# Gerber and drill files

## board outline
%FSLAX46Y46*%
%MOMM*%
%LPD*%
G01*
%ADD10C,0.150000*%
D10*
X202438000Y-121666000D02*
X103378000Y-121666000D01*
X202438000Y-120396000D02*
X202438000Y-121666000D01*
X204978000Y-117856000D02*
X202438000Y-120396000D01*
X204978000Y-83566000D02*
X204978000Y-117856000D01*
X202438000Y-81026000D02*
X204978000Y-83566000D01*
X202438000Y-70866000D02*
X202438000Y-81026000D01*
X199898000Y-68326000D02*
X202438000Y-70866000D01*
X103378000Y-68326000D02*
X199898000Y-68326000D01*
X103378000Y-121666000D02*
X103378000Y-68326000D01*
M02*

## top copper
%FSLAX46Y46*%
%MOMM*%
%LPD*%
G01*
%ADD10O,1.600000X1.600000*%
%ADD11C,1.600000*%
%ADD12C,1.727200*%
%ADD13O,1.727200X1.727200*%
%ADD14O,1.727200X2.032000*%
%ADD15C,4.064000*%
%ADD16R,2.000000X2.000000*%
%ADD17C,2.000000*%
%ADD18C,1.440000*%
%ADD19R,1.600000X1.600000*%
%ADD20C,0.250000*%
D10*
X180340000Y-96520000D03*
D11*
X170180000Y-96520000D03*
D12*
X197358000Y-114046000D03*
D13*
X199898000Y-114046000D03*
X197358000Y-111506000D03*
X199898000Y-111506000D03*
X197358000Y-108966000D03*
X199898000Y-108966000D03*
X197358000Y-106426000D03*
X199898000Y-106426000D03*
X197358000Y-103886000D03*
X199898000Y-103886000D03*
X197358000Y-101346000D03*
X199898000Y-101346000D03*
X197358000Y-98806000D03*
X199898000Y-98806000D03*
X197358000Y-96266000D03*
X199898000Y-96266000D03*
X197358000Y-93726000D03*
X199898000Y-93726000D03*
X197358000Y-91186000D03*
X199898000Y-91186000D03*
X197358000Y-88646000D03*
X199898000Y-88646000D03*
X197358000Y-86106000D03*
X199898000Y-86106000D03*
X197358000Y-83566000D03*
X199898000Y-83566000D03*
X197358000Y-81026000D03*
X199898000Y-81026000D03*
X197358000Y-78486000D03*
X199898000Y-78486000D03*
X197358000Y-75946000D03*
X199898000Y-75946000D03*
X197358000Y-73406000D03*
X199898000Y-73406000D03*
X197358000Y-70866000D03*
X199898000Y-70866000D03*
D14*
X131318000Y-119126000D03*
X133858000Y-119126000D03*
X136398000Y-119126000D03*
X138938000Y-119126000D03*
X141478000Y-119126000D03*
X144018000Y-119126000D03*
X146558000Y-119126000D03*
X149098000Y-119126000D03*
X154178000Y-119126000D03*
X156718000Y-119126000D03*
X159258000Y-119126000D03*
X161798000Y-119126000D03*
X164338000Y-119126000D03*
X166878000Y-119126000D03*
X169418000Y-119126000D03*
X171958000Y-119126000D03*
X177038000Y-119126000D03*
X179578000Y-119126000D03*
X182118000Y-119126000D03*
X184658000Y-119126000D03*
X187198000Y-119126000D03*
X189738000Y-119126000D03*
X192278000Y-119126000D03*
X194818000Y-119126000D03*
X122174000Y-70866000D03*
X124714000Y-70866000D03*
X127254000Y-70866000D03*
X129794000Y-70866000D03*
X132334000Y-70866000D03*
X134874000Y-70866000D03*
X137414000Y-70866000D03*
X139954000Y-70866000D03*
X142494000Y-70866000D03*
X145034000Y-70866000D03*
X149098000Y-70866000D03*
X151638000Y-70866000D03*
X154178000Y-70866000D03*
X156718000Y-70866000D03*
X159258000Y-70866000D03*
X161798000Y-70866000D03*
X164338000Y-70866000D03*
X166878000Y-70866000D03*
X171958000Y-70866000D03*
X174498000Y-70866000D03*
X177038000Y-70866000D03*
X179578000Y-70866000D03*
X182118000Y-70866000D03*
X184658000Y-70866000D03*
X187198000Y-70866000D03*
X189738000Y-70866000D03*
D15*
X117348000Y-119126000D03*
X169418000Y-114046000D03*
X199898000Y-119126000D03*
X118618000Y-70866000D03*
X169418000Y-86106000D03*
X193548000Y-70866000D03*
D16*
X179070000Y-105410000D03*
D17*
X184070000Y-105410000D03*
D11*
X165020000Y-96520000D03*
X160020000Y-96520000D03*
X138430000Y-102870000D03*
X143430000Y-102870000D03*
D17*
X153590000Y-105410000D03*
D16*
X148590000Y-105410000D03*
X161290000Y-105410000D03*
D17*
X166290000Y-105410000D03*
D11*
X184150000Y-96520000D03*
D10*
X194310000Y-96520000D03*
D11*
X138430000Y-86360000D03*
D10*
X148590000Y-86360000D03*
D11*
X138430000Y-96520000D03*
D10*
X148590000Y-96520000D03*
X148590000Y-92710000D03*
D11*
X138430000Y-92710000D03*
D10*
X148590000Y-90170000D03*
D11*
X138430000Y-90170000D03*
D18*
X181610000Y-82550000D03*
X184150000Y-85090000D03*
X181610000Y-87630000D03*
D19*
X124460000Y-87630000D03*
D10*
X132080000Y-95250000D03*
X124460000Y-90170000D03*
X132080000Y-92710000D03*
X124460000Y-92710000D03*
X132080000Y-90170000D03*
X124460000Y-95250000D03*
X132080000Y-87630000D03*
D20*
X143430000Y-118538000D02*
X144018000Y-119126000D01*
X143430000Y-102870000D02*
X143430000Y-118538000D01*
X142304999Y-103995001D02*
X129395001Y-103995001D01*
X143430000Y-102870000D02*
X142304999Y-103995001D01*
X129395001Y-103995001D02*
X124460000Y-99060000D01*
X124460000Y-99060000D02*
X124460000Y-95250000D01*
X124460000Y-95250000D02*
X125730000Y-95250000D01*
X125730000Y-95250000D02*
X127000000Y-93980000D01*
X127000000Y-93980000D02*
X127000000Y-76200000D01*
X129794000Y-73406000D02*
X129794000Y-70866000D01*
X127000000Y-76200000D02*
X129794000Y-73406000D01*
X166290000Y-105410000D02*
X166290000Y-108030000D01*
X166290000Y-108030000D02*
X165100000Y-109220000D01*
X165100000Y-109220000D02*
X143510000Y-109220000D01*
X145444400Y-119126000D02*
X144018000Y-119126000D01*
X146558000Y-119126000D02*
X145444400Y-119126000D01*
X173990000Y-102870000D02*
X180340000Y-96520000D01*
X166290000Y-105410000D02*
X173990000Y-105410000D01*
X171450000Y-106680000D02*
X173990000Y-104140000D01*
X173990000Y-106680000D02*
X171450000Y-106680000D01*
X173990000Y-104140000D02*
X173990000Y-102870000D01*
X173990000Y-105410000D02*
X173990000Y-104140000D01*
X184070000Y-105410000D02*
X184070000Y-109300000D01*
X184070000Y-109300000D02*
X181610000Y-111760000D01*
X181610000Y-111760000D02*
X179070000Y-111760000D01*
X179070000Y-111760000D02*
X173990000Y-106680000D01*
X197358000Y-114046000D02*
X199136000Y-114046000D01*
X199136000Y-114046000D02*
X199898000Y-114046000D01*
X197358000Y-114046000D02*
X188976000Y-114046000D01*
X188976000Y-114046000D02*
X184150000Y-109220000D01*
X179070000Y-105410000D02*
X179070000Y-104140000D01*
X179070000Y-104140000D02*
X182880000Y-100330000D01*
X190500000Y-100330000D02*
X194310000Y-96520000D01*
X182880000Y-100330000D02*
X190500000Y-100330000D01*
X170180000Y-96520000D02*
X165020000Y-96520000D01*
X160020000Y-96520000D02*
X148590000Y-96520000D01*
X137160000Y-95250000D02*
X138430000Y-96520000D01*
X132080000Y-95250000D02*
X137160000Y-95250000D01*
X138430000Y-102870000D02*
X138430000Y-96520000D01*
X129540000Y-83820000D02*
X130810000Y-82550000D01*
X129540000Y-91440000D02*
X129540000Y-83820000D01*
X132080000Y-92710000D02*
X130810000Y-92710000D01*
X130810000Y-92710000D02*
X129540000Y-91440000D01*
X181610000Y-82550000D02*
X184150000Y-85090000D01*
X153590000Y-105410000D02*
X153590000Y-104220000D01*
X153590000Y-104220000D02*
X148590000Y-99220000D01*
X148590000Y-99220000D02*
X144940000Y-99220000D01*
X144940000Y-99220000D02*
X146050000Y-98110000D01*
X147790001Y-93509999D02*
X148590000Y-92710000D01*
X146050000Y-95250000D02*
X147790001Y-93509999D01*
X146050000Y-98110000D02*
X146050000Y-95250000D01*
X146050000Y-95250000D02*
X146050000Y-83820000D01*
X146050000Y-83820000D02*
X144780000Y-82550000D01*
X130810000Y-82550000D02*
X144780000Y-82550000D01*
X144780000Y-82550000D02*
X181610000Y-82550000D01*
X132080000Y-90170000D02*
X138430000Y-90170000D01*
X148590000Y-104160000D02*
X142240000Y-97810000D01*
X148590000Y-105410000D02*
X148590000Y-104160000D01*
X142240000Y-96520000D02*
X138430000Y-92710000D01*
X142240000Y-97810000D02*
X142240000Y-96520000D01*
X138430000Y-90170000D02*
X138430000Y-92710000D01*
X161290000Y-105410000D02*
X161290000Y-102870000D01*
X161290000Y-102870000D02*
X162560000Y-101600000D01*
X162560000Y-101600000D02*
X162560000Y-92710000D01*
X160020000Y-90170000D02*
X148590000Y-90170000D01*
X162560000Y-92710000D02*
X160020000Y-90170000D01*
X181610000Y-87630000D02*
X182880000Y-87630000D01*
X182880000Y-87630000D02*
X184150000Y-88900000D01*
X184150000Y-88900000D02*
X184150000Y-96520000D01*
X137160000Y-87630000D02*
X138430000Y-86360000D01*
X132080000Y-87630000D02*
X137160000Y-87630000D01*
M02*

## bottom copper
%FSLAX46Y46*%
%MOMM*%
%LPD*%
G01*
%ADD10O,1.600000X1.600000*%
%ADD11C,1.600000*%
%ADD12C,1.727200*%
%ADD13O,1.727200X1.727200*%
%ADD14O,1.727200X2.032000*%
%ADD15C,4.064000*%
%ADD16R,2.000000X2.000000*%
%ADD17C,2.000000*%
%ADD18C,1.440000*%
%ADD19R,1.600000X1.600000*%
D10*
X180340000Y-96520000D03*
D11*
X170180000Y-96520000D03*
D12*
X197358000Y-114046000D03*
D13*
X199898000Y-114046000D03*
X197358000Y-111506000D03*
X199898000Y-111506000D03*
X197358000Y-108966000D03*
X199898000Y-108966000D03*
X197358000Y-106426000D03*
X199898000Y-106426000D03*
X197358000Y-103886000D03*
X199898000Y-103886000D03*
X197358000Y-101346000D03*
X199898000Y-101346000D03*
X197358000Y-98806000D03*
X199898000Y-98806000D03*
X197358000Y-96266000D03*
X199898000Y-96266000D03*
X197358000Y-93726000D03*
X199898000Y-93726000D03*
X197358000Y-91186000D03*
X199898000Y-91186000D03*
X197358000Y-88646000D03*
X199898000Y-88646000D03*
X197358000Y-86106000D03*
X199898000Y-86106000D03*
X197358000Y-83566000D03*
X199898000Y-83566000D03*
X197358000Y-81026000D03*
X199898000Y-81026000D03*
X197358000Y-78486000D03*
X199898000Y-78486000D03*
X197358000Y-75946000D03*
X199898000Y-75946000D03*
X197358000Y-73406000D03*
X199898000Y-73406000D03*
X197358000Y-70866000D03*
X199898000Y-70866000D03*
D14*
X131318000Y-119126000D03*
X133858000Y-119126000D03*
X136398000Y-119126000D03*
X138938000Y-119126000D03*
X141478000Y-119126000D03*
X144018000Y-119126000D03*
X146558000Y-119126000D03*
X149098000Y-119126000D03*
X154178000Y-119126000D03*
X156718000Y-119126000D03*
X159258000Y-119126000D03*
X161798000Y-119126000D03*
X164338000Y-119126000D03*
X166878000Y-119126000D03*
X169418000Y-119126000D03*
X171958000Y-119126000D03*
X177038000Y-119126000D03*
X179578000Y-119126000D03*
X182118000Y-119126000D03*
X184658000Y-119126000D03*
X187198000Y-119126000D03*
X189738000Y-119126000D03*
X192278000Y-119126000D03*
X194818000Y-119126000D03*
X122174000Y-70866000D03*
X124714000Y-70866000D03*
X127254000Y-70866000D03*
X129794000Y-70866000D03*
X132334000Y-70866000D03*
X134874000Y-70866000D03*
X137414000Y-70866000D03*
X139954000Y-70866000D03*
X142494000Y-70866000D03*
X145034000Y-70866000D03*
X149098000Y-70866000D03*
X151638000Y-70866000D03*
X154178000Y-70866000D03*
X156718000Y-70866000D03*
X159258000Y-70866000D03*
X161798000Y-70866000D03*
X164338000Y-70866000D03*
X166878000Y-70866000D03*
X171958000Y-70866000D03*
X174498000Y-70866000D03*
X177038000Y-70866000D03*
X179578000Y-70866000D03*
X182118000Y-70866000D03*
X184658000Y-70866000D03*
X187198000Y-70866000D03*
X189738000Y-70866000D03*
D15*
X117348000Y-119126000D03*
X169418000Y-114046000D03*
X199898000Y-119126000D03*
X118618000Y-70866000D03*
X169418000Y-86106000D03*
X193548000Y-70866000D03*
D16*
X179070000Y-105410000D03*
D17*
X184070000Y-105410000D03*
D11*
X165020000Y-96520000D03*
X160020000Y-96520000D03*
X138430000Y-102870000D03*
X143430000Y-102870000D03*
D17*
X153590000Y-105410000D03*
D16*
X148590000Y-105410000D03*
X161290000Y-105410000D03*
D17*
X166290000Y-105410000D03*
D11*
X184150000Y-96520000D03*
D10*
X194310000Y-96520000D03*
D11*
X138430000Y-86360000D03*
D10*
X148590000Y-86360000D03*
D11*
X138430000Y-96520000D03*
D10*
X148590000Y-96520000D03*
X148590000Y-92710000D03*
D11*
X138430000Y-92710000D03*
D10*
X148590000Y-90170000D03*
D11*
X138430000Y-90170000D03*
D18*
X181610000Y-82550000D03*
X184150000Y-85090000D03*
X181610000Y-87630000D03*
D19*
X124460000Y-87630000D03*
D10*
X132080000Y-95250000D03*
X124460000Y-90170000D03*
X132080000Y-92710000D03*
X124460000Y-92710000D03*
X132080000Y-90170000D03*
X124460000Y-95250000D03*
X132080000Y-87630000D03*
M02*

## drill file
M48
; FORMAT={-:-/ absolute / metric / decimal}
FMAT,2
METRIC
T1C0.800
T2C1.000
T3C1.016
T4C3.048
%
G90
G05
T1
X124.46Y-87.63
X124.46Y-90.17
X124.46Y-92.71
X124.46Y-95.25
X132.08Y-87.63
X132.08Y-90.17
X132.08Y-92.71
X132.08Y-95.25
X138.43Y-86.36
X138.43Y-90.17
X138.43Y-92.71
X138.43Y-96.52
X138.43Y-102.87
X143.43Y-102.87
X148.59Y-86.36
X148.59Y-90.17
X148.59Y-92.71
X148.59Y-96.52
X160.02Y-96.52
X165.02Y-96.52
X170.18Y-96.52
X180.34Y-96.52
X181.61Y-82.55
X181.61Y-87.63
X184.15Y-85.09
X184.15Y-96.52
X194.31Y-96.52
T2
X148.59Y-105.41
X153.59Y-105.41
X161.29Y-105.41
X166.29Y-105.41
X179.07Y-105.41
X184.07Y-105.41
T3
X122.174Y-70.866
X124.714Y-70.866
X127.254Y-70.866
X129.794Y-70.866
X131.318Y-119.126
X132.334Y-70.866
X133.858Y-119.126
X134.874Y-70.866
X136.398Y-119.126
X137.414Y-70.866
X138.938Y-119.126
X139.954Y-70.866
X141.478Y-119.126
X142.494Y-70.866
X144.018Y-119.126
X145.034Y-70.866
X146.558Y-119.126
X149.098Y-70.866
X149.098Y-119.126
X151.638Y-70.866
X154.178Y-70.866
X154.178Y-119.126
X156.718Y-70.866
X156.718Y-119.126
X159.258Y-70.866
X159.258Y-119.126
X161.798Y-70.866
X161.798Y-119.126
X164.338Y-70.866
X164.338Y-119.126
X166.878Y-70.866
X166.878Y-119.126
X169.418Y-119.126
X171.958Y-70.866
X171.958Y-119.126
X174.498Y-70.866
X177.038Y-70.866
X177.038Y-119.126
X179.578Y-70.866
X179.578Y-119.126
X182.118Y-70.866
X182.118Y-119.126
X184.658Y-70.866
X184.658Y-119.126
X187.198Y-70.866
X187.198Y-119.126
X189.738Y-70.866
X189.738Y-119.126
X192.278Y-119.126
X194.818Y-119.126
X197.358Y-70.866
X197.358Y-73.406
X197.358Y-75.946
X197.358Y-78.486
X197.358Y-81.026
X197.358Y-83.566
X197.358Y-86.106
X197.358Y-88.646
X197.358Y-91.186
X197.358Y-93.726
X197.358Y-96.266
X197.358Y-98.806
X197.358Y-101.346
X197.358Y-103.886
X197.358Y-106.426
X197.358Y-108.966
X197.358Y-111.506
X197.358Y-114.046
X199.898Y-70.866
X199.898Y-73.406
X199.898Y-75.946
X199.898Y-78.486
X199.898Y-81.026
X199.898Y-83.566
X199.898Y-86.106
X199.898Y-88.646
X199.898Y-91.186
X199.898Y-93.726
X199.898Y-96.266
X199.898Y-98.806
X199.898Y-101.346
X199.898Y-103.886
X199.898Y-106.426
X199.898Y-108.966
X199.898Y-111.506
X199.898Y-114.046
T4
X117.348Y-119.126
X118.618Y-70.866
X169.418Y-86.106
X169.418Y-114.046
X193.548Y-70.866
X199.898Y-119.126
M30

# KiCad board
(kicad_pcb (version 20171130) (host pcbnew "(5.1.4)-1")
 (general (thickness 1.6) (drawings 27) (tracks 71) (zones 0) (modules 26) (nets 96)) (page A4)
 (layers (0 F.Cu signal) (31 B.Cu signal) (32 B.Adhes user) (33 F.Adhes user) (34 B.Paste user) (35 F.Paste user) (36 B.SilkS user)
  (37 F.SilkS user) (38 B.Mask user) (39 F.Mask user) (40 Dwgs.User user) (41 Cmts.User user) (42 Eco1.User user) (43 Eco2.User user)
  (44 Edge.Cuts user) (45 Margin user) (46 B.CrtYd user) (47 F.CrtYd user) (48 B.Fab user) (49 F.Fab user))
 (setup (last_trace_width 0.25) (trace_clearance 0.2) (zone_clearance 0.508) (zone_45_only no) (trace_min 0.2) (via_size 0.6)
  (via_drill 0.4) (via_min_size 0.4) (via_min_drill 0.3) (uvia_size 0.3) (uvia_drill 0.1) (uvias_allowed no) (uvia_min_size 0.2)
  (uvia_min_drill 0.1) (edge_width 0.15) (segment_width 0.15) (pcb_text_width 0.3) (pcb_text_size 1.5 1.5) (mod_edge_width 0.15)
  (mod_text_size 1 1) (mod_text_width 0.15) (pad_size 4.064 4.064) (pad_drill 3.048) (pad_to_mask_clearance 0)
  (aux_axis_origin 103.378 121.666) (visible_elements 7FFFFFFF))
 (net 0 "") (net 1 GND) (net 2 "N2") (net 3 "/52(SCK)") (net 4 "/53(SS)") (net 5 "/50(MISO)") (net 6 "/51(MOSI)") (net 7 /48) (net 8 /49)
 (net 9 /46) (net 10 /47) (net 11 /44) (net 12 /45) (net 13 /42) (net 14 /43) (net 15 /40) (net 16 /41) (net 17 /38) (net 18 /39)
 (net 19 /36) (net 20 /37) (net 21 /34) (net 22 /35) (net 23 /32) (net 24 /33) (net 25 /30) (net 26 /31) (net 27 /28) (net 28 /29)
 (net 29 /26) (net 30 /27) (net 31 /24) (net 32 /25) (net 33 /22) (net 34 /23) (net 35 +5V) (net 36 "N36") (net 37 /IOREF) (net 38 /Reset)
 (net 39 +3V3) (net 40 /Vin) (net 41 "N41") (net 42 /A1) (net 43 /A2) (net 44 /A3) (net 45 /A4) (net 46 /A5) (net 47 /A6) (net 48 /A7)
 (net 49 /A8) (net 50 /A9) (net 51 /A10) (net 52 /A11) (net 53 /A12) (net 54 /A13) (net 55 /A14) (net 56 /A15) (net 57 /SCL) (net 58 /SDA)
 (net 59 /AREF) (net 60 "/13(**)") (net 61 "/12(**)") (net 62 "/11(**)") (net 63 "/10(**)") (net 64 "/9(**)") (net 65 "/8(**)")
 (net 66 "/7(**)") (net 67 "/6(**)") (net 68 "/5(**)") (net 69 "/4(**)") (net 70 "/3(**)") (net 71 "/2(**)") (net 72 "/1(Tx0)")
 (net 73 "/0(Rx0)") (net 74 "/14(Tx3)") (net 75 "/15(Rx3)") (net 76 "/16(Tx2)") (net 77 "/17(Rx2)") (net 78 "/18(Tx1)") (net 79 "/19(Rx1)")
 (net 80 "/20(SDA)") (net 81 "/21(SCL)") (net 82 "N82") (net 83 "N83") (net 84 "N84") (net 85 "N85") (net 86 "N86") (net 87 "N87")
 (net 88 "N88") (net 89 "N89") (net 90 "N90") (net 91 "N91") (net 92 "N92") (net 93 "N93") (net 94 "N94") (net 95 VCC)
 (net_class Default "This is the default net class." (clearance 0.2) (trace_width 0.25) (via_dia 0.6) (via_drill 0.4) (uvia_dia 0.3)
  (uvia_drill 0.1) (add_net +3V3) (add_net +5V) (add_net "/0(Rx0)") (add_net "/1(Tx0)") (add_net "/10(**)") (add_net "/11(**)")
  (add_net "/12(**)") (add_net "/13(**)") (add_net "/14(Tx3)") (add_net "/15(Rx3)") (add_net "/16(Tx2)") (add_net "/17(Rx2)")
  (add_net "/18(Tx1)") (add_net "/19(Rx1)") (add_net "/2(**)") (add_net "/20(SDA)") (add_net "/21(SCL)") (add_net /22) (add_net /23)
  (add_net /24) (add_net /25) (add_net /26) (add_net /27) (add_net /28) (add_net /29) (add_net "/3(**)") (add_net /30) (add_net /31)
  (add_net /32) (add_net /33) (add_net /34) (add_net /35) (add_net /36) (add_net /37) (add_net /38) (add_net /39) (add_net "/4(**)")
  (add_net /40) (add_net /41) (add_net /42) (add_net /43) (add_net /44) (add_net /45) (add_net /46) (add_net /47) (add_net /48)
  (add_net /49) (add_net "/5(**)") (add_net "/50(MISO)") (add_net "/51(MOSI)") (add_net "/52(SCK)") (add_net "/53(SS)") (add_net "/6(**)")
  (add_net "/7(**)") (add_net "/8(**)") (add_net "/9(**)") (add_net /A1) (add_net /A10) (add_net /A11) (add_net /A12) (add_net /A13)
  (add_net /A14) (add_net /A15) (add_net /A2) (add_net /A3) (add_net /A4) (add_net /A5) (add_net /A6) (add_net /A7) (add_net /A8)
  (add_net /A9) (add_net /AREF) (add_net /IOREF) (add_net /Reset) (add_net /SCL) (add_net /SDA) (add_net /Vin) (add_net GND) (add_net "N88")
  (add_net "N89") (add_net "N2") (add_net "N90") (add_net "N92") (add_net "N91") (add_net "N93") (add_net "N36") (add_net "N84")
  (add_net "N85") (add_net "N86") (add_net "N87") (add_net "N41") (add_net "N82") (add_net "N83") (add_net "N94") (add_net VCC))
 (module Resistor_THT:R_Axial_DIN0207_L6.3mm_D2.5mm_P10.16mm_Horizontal (layer F.Cu) (at 170.18 96.52)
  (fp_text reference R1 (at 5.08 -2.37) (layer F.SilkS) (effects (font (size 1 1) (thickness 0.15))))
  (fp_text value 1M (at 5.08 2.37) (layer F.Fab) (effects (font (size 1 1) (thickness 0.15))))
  (pad 2 thru_hole oval (at 10.16 0) (size 1.6 1.6) (drill 0.8) (layers *.Cu *.Mask) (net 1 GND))
  (pad 1 thru_hole circle (at 0 0) (size 1.6 1.6) (drill 0.8) (layers *.Cu *.Mask) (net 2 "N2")))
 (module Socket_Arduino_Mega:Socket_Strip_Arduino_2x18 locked (layer F.Cu) (at 197.358 114.046 90)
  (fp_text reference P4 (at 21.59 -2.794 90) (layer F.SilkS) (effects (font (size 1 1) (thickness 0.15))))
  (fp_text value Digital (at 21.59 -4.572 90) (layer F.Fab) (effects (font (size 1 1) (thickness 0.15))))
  (pad 1 thru_hole circle (at 0 0 90) (size 1.7272 1.7272) (drill 1.016) (layers *.Cu *.Mask F.SilkS) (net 1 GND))
  (pad 2 thru_hole oval (at 0 2.54 90) (size 1.7272 1.7272) (drill 1.016) (layers *.Cu *.Mask F.SilkS) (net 1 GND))
  (pad 3 thru_hole oval (at 2.54 0 90) (size 1.7272 1.7272) (drill 1.016) (layers *.Cu *.Mask F.SilkS) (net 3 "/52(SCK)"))
  (pad 4 thru_hole oval (at 2.54 2.54 90) (size 1.7272 1.7272) (drill 1.016) (layers *.Cu *.Mask F.SilkS) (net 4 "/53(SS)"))
  (pad 5 thru_hole oval (at 5.08 0 90) (size 1.7272 1.7272) (drill 1.016) (layers *.Cu *.Mask F.SilkS) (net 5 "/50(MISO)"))
  (pad 6 thru_hole oval (at 5.08 2.54 90) (size 1.7272 1.7272) (drill 1.016) (layers *.Cu *.Mask F.SilkS) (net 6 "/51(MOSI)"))
  (pad 7 thru_hole oval (at 7.62 0 90) (size 1.7272 1.7272) (drill 1.016) (layers *.Cu *.Mask F.SilkS) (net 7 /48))
  (pad 8 thru_hole oval (at 7.62 2.54 90) (size 1.7272 1.7272) (drill 1.016) (layers *.Cu *.Mask F.SilkS) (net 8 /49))
  (pad 9 thru_hole oval (at 10.16 0 90) (size 1.7272 1.7272) (drill 1.016) (layers *.Cu *.Mask F.SilkS) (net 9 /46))
  (pad 10 thru_hole oval (at 10.16 2.54 90) (size 1.7272 1.7272) (drill 1.016) (layers *.Cu *.Mask F.SilkS) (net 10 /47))
  (pad 11 thru_hole oval (at 12.7 0 90) (size 1.7272 1.7272) (drill 1.016) (layers *.Cu *.Mask F.SilkS) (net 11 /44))
  (pad 12 thru_hole oval (at 12.7 2.54 90) (size 1.7272 1.7272) (drill 1.016) (layers *.Cu *.Mask F.SilkS) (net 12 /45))
  (pad 13 thru_hole oval (at 15.24 0 90) (size 1.7272 1.7272) (drill 1.016) (layers *.Cu *.Mask F.SilkS) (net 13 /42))
  (pad 14 thru_hole oval (at 15.24 2.54 90) (size 1.7272 1.7272) (drill 1.016) (layers *.Cu *.Mask F.SilkS) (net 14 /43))
  (pad 15 thru_hole oval (at 17.78 0 90) (size 1.7272 1.7272) (drill 1.016) (layers *.Cu *.Mask F.SilkS) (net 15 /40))
  (pad 16 thru_hole oval (at 17.78 2.54 90) (size 1.7272 1.7272) (drill 1.016) (layers *.Cu *.Mask F.SilkS) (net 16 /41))
  (pad 17 thru_hole oval (at 20.32 0 90) (size 1.7272 1.7272) (drill 1.016) (layers *.Cu *.Mask F.SilkS) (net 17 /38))
  (pad 18 thru_hole oval (at 20.32 2.54 90) (size 1.7272 1.7272) (drill 1.016) (layers *.Cu *.Mask F.SilkS) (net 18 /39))
  (pad 19 thru_hole oval (at 22.86 0 90) (size 1.7272 1.7272) (drill 1.016) (layers *.Cu *.Mask F.SilkS) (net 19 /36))
  (pad 20 thru_hole oval (at 22.86 2.54 90) (size 1.7272 1.7272) (drill 1.016) (layers *.Cu *.Mask F.SilkS) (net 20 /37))
  (pad 21 thru_hole oval (at 25.4 0 90) (size 1.7272 1.7272) (drill 1.016) (layers *.Cu *.Mask F.SilkS) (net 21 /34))
  (pad 22 thru_hole oval (at 25.4 2.54 90) (size 1.7272 1.7272) (drill 1.016) (layers *.Cu *.Mask F.SilkS) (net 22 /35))
  (pad 23 thru_hole oval (at 27.94 0 90) (size 1.7272 1.7272) (drill 1.016) (layers *.Cu *.Mask F.SilkS) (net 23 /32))
  (pad 24 thru_hole oval (at 27.94 2.54 90) (size 1.7272 1.7272) (drill 1.016) (layers *.Cu *.Mask F.SilkS) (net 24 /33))
  (pad 25 thru_hole oval (at 30.48 0 90) (size 1.7272 1.7272) (drill 1.016) (layers *.Cu *.Mask F.SilkS) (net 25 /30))
  (pad 26 thru_hole oval (at 30.48 2.54 90) (size 1.7272 1.7272) (drill 1.016) (layers *.Cu *.Mask F.SilkS) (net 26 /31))
  (pad 27 thru_hole oval (at 33.02 0 90) (size 1.7272 1.7272) (drill 1.016) (layers *.Cu *.Mask F.SilkS) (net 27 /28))
  (pad 28 thru_hole oval (at 33.02 2.54 90) (size 1.7272 1.7272) (drill 1.016) (layers *.Cu *.Mask F.SilkS) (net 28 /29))
  (pad 29 thru_hole oval (at 35.56 0 90) (size 1.7272 1.7272) (drill 1.016) (layers *.Cu *.Mask F.SilkS) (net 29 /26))
  (pad 30 thru_hole oval (at 35.56 2.54 90) (size 1.7272 1.7272) (drill 1.016) (layers *.Cu *.Mask F.SilkS) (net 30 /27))
  (pad 31 thru_hole oval (at 38.1 0 90) (size 1.7272 1.7272) (drill 1.016) (layers *.Cu *.Mask F.SilkS) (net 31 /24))
  (pad 32 thru_hole oval (at 38.1 2.54 90) (size 1.7272 1.7272) (drill 1.016) (layers *.Cu *.Mask F.SilkS) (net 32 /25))
  (pad 33 thru_hole oval (at 40.64 0 90) (size 1.7272 1.7272) (drill 1.016) (layers *.Cu *.Mask F.SilkS) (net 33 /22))
  (pad 34 thru_hole oval (at 40.64 2.54 90) (size 1.7272 1.7272) (drill 1.016) (layers *.Cu *.Mask F.SilkS) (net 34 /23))
  (pad 35 thru_hole oval (at 43.18 0 90) (size 1.7272 1.7272) (drill 1.016) (layers *.Cu *.Mask F.SilkS) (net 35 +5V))
  (pad 36 thru_hole oval (at 43.18 2.54 90) (size 1.7272 1.7272) (drill 1.016) (layers *.Cu *.Mask F.SilkS) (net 35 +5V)))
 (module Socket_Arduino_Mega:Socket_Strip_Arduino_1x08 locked (layer F.Cu) (at 131.318 119.126)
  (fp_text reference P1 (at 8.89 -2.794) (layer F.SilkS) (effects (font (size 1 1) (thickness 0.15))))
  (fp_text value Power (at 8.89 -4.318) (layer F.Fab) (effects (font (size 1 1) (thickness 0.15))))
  (pad 1 thru_hole oval (at 0 0) (size 1.7272 2.032) (drill 1.016) (layers *.Cu *.Mask F.SilkS) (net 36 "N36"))
  (pad 2 thru_hole oval (at 2.54 0) (size 1.7272 2.032) (drill 1.016) (layers *.Cu *.Mask F.SilkS) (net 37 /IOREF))
  (pad 3 thru_hole oval (at 5.08 0) (size 1.7272 2.032) (drill 1.016) (layers *.Cu *.Mask F.SilkS) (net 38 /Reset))
  (pad 4 thru_hole oval (at 7.62 0) (size 1.7272 2.032) (drill 1.016) (layers *.Cu *.Mask F.SilkS) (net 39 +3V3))
  (pad 5 thru_hole oval (at 10.16 0) (size 1.7272 2.032) (drill 1.016) (layers *.Cu *.Mask F.SilkS) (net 35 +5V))
  (pad 6 thru_hole oval (at 12.7 0) (size 1.7272 2.032) (drill 1.016) (layers *.Cu *.Mask F.SilkS) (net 1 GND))
  (pad 7 thru_hole oval (at 15.24 0) (size 1.7272 2.032) (drill 1.016) (layers *.Cu *.Mask F.SilkS) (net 1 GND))
  (pad 8 thru_hole oval (at 17.78 0) (size 1.7272 2.032) (drill 1.016) (layers *.Cu *.Mask F.SilkS) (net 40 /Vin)))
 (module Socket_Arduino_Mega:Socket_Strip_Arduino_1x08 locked (layer F.Cu) (at 154.178 119.126)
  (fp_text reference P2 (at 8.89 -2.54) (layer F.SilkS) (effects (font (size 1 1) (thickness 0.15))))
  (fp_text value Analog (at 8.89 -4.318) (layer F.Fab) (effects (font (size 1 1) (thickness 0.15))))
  (pad 1 thru_hole oval (at 0 0) (size 1.7272 2.032) (drill 1.016) (layers *.Cu *.Mask F.SilkS) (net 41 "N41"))
  (pad 2 thru_hole oval (at 2.54 0) (size 1.7272 2.032) (drill 1.016) (layers *.Cu *.Mask F.SilkS) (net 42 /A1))
  (pad 3 thru_hole oval (at 5.08 0) (size 1.7272 2.032) (drill 1.016) (layers *.Cu *.Mask F.SilkS) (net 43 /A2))
  (pad 4 thru_hole oval (at 7.62 0) (size 1.7272 2.032) (drill 1.016) (layers *.Cu *.Mask F.SilkS) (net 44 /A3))
  (pad 5 thru_hole oval (at 10.16 0) (size 1.7272 2.032) (drill 1.016) (layers *.Cu *.Mask F.SilkS) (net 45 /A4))
  (pad 6 thru_hole oval (at 12.7 0) (size 1.7272 2.032) (drill 1.016) (layers *.Cu *.Mask F.SilkS) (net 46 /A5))
  (pad 7 thru_hole oval (at 15.24 0) (size 1.7272 2.032) (drill 1.016) (layers *.Cu *.Mask F.SilkS) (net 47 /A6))
  (pad 8 thru_hole oval (at 17.78 0) (size 1.7272 2.032) (drill 1.016) (layers *.Cu *.Mask F.SilkS) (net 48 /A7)))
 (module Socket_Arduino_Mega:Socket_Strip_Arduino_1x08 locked (layer F.Cu) (at 177.038 119.126)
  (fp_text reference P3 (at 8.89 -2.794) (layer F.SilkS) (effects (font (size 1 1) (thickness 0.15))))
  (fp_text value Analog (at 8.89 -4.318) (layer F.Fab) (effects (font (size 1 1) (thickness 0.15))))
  (pad 1 thru_hole oval (at 0 0) (size 1.7272 2.032) (drill 1.016) (layers *.Cu *.Mask F.SilkS) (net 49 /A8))
  (pad 2 thru_hole oval (at 2.54 0) (size 1.7272 2.032) (drill 1.016) (layers *.Cu *.Mask F.SilkS) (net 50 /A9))
  (pad 3 thru_hole oval (at 5.08 0) (size 1.7272 2.032) (drill 1.016) (layers *.Cu *.Mask F.SilkS) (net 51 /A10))
  (pad 4 thru_hole oval (at 7.62 0) (size 1.7272 2.032) (drill 1.016) (layers *.Cu *.Mask F.SilkS) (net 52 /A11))
  (pad 5 thru_hole oval (at 10.16 0) (size 1.7272 2.032) (drill 1.016) (layers *.Cu *.Mask F.SilkS) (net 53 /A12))
  (pad 6 thru_hole oval (at 12.7 0) (size 1.7272 2.032) (drill 1.016) (layers *.Cu *.Mask F.SilkS) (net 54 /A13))
  (pad 7 thru_hole oval (at 15.24 0) (size 1.7272 2.032) (drill 1.016) (layers *.Cu *.Mask F.SilkS) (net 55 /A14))
  (pad 8 thru_hole oval (at 17.78 0) (size 1.7272 2.032) (drill 1.016) (layers *.Cu *.Mask F.SilkS) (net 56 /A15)))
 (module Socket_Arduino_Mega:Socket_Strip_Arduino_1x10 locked (layer F.Cu) (at 122.174 70.866)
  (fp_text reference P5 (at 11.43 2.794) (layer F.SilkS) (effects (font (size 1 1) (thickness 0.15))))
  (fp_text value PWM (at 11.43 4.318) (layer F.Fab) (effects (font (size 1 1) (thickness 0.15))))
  (pad 1 thru_hole oval (at 0 0) (size 1.7272 2.032) (drill 1.016) (layers *.Cu *.Mask F.SilkS) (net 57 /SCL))
  (pad 2 thru_hole oval (at 2.54 0) (size 1.7272 2.032) (drill 1.016) (layers *.Cu *.Mask F.SilkS) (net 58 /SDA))
  (pad 3 thru_hole oval (at 5.08 0) (size 1.7272 2.032) (drill 1.016) (layers *.Cu *.Mask F.SilkS) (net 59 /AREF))
  (pad 4 thru_hole oval (at 7.62 0) (size 1.7272 2.032) (drill 1.016) (layers *.Cu *.Mask F.SilkS) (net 1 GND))
  (pad 5 thru_hole oval (at 10.16 0) (size 1.7272 2.032) (drill 1.016) (layers *.Cu *.Mask F.SilkS) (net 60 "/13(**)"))
  (pad 6 thru_hole oval (at 12.7 0) (size 1.7272 2.032) (drill 1.016) (layers *.Cu *.Mask F.SilkS) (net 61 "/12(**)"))
  (pad 7 thru_hole oval (at 15.24 0) (size 1.7272 2.032) (drill 1.016) (layers *.Cu *.Mask F.SilkS) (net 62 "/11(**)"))
  (pad 8 thru_hole oval (at 17.78 0) (size 1.7272 2.032) (drill 1.016) (layers *.Cu *.Mask F.SilkS) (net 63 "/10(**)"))
  (pad 9 thru_hole oval (at 20.32 0) (size 1.7272 2.032) (drill 1.016) (layers *.Cu *.Mask F.SilkS) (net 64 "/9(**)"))
  (pad 10 thru_hole oval (at 22.86 0) (size 1.7272 2.032) (drill 1.016) (layers *.Cu *.Mask F.SilkS) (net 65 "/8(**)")))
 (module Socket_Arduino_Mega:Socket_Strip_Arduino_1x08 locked (layer F.Cu) (at 149.098 70.866)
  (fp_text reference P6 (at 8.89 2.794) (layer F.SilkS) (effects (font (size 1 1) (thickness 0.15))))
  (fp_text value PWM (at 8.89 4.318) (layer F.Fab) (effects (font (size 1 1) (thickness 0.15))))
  (pad 1 thru_hole oval (at 0 0) (size 1.7272 2.032) (drill 1.016) (layers *.Cu *.Mask F.SilkS) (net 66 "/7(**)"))
  (pad 2 thru_hole oval (at 2.54 0) (size 1.7272 2.032) (drill 1.016) (layers *.Cu *.Mask F.SilkS) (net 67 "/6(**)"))
  (pad 3 thru_hole oval (at 5.08 0) (size 1.7272 2.032) (drill 1.016) (layers *.Cu *.Mask F.SilkS) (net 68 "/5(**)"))
  (pad 4 thru_hole oval (at 7.62 0) (size 1.7272 2.032) (drill 1.016) (layers *.Cu *.Mask F.SilkS) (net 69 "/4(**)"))
  (pad 5 thru_hole oval (at 10.16 0) (size 1.7272 2.032) (drill 1.016) (layers *.Cu *.Mask F.SilkS) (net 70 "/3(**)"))
  (pad 6 thru_hole oval (at 12.7 0) (size 1.7272 2.032) (drill 1.016) (layers *.Cu *.Mask F.SilkS) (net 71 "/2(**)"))
  (pad 7 thru_hole oval (at 15.24 0) (size 1.7272 2.032) (drill 1.016) (layers *.Cu *.Mask F.SilkS) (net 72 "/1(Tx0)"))
  (pad 8 thru_hole oval (at 17.78 0) (size 1.7272 2.032) (drill 1.016) (layers *.Cu *.Mask F.SilkS) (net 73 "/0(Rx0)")))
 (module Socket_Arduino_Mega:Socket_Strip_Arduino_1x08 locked (layer F.Cu) (at 171.958 70.866)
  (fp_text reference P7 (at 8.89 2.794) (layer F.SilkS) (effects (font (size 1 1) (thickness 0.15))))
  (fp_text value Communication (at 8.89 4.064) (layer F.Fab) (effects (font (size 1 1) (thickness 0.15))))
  (pad 1 thru_hole oval (at 0 0) (size 1.7272 2.032) (drill 1.016) (layers *.Cu *.Mask F.SilkS) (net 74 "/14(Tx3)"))
  (pad 2 thru_hole oval (at 2.54 0) (size 1.7272 2.032) (drill 1.016) (layers *.Cu *.Mask F.SilkS) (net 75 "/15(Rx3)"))
  (pad 3 thru_hole oval (at 5.08 0) (size 1.7272 2.032) (drill 1.016) (layers *.Cu *.Mask F.SilkS) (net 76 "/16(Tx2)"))
  (pad 4 thru_hole oval (at 7.62 0) (size 1.7272 2.032) (drill 1.016) (layers *.Cu *.Mask F.SilkS) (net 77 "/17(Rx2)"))
  (pad 5 thru_hole oval (at 10.16 0) (size 1.7272 2.032) (drill 1.016) (layers *.Cu *.Mask F.SilkS) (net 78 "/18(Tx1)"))
  (pad 6 thru_hole oval (at 12.7 0) (size 1.7272 2.032) (drill 1.016) (layers *.Cu *.Mask F.SilkS) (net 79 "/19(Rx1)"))
  (pad 7 thru_hole oval (at 15.24 0) (size 1.7272 2.032) (drill 1.016) (layers *.Cu *.Mask F.SilkS) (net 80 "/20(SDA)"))
  (pad 8 thru_hole oval (at 17.78 0) (size 1.7272 2.032) (drill 1.016) (layers *.Cu *.Mask F.SilkS) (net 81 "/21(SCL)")))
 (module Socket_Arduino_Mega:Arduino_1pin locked (layer F.Cu) (at 117.348 119.126)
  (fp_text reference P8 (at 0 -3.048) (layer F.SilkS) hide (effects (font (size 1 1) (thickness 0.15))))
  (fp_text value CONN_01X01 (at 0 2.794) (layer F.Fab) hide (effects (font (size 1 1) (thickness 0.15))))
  (pad 1 thru_hole circle (at 0 0) (size 4.064 4.064) (drill 3.048) (layers *.Cu *.Mask F.SilkS) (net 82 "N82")))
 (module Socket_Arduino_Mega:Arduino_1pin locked (layer F.Cu) (at 169.418 114.046)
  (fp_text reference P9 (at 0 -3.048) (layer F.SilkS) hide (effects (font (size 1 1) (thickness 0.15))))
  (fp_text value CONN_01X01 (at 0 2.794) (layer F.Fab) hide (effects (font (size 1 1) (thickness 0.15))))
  (pad 1 thru_hole circle (at 0 0) (size 4.064 4.064) (drill 3.048) (layers *.Cu *.Mask F.SilkS) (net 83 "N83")))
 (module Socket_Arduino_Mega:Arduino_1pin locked (layer F.Cu) (at 199.898 119.126)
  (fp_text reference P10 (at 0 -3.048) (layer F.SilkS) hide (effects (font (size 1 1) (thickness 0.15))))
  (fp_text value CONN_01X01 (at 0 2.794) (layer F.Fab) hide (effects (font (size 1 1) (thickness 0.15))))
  (pad 1 thru_hole circle (at 0 0) (size 4.064 4.064) (drill 3.048) (layers *.Cu *.Mask F.SilkS) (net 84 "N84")))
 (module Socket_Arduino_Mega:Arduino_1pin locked (layer F.Cu) (at 118.618 70.866)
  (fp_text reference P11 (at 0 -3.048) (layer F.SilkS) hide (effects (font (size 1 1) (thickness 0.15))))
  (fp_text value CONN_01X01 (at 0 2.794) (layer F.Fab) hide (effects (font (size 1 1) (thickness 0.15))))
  (pad 1 thru_hole circle (at 0 0) (size 4.064 4.064) (drill 3.048) (layers *.Cu *.Mask F.SilkS) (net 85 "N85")))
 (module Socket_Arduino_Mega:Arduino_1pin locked (layer F.Cu) (at 169.418 86.106)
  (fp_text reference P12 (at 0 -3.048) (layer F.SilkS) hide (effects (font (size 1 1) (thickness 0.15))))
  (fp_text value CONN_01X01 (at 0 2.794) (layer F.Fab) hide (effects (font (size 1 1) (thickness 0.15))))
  (pad 1 thru_hole circle (at 0 0) (size 4.064 4.064) (drill 3.048) (layers *.Cu *.Mask F.SilkS) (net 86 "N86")))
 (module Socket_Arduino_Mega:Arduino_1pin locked (layer F.Cu) (at 193.548 70.866)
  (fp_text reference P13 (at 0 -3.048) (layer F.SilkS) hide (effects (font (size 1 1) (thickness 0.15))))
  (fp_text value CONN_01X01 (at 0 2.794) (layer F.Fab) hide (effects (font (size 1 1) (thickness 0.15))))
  (pad 1 thru_hole circle (at 0 0) (size 4.064 4.064) (drill 3.048) (layers *.Cu *.Mask F.SilkS) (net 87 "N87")))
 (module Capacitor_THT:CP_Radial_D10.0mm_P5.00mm (layer F.Cu) (at 179.07 105.41)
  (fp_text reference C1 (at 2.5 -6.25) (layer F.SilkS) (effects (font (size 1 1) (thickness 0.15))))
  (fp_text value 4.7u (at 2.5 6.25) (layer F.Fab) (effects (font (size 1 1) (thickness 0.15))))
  (pad 1 thru_hole rect (at 0 0) (size 2 2) (drill 1) (layers *.Cu *.Mask) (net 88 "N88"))
  (pad 2 thru_hole circle (at 5 0) (size 2 2) (drill 1) (layers *.Cu *.Mask) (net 1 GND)))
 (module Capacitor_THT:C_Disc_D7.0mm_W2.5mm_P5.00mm (layer F.Cu) (at 160.02 96.52)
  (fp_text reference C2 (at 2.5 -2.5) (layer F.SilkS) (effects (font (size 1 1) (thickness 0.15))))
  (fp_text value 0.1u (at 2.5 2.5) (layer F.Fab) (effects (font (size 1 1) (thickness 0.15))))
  (pad 2 thru_hole circle (at 5 0) (size 1.6 1.6) (drill 0.8) (layers *.Cu *.Mask) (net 2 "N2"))
  (pad 1 thru_hole circle (at 0 0) (size 1.6 1.6) (drill 0.8) (layers *.Cu *.Mask) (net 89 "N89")))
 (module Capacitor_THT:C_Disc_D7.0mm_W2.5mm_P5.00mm (layer F.Cu) (at 138.43 102.87)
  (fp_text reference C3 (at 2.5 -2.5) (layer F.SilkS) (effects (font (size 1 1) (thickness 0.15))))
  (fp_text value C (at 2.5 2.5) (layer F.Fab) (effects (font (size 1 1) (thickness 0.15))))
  (pad 1 thru_hole circle (at 0 0) (size 1.6 1.6) (drill 0.8) (layers *.Cu *.Mask) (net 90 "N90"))
  (pad 2 thru_hole circle (at 5 0) (size 1.6 1.6) (drill 0.8) (layers *.Cu *.Mask) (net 1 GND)))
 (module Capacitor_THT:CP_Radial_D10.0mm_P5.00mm (layer F.Cu) (at 148.59 105.41)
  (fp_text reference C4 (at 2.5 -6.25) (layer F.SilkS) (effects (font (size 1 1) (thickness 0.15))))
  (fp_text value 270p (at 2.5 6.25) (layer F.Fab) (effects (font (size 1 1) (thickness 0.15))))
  (pad 2 thru_hole circle (at 5 0) (size 2 2) (drill 1) (layers *.Cu *.Mask) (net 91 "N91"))
  (pad 1 thru_hole rect (at 0 0) (size 2 2) (drill 1) (layers *.Cu *.Mask) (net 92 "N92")))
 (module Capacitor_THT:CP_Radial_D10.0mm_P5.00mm (layer F.Cu) (at 161.29 105.41)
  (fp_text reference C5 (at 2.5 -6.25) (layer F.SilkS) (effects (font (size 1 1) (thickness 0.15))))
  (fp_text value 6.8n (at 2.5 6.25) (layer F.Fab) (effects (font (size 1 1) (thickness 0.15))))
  (pad 1 thru_hole rect (at 0 0) (size 2 2) (drill 1) (layers *.Cu *.Mask) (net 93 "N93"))
  (pad 2 thru_hole circle (at 5 0) (size 2 2) (drill 1) (layers *.Cu *.Mask) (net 1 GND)))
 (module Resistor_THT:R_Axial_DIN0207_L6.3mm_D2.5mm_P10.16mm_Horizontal (layer F.Cu) (at 184.15 96.52)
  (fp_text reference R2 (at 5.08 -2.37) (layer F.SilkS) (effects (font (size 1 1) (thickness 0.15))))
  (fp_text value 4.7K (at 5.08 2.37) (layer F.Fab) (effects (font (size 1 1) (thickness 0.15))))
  (pad 1 thru_hole circle (at 0 0) (size 1.6 1.6) (drill 0.8) (layers *.Cu *.Mask) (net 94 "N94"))
  (pad 2 thru_hole oval (at 10.16 0) (size 1.6 1.6) (drill 0.8) (layers *.Cu *.Mask) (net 88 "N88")))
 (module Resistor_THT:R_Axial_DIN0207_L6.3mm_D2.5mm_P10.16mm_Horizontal (layer F.Cu) (at 138.43 86.36)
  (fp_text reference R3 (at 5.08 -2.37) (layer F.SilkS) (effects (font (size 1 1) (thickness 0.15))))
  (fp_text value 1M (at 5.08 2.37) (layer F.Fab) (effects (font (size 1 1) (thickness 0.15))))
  (pad 1 thru_hole circle (at 0 0) (size 1.6 1.6) (drill 0.8) (layers *.Cu *.Mask) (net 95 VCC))
  (pad 2 thru_hole oval (at 10.16 0) (size 1.6 1.6) (drill 0.8) (layers *.Cu *.Mask) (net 89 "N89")))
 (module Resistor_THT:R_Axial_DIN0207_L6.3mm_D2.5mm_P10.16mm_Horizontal (layer F.Cu) (at 138.43 96.52)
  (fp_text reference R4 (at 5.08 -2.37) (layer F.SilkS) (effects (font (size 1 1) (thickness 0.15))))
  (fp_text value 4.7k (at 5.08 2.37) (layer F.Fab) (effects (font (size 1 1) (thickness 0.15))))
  (pad 1 thru_hole circle (at 0 0) (size 1.6 1.6) (drill 0.8) (layers *.Cu *.Mask) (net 90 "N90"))
  (pad 2 thru_hole oval (at 10.16 0) (size 1.6 1.6) (drill 0.8) (layers *.Cu *.Mask) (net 89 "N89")))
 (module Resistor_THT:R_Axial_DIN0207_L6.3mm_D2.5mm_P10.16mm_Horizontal (layer F.Cu) (at 138.43 92.71)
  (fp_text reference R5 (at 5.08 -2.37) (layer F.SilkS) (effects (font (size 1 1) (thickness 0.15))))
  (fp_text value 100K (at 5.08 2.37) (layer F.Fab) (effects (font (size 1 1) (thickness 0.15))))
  (pad 2 thru_hole oval (at 10.16 0) (size 1.6 1.6) (drill 0.8) (layers *.Cu *.Mask) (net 91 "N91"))
  (pad 1 thru_hole circle (at 0 0) (size 1.6 1.6) (drill 0.8) (layers *.Cu *.Mask) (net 92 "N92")))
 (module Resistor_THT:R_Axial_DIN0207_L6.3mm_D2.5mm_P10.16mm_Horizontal (layer F.Cu) (at 138.43 90.17)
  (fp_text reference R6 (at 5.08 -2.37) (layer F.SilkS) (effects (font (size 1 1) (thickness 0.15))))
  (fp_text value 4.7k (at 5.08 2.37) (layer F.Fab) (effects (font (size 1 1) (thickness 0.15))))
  (pad 2 thru_hole oval (at 10.16 0) (size 1.6 1.6) (drill 0.8) (layers *.Cu *.Mask) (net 93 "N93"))
  (pad 1 thru_hole circle (at 0 0) (size 1.6 1.6) (drill 0.8) (layers *.Cu *.Mask) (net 92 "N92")))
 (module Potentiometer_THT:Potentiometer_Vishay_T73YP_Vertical (layer F.Cu) (at 181.61 87.63)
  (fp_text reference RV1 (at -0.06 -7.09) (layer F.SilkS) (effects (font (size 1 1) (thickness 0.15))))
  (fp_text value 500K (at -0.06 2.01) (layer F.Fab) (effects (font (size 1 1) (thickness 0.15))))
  (pad 3 thru_hole circle (at 0 -5.08) (size 1.44 1.44) (drill 0.8) (layers *.Cu *.Mask) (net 91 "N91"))
  (pad 2 thru_hole circle (at 2.54 -2.54) (size 1.44 1.44) (drill 0.8) (layers *.Cu *.Mask) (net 91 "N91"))
  (pad 1 thru_hole circle (at 0 0) (size 1.44 1.44) (drill 0.8) (layers *.Cu *.Mask) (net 94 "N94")))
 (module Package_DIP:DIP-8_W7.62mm (layer F.Cu) (at 124.46 87.63)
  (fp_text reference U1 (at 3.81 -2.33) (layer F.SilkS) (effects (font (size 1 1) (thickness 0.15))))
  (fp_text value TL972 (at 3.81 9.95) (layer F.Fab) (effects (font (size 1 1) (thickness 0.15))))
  (pad 1 thru_hole rect (at 0 0) (size 1.6 1.6) (drill 0.8) (layers *.Cu *.Mask))
  (pad 5 thru_hole oval (at 7.62 7.62) (size 1.6 1.6) (drill 0.8) (layers *.Cu *.Mask) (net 90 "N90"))
  (pad 2 thru_hole oval (at 0 2.54) (size 1.6 1.6) (drill 0.8) (layers *.Cu *.Mask))
  (pad 6 thru_hole oval (at 7.62 5.08) (size 1.6 1.6) (drill 0.8) (layers *.Cu *.Mask) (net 91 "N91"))
  (pad 3 thru_hole oval (at 0 5.08) (size 1.6 1.6) (drill 0.8) (layers *.Cu *.Mask))
  (pad 7 thru_hole oval (at 7.62 2.54) (size 1.6 1.6) (drill 0.8) (layers *.Cu *.Mask) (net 92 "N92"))
  (pad 4 thru_hole oval (at 0 7.62) (size 1.6 1.6) (drill 0.8) (layers *.Cu *.Mask) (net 1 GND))
  (pad 8 thru_hole oval (at 7.62 0) (size 1.6 1.6) (drill 0.8) (layers *.Cu *.Mask) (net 95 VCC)))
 (gr_line (start 202.438 121.666) (end 103.378 121.666) (angle 90) (layer Edge.Cuts) (width 0.15))
 (gr_line (start 202.438 120.396) (end 202.438 121.666) (angle 90) (layer Edge.Cuts) (width 0.15))
 (gr_line (start 204.978 117.856) (end 202.438 120.396) (angle 90) (layer Edge.Cuts) (width 0.15))
 (gr_line (start 204.978 83.566) (end 204.978 117.856) (angle 90) (layer Edge.Cuts) (width 0.15))
 (gr_line (start 202.438 81.026) (end 204.978 83.566) (angle 90) (layer Edge.Cuts) (width 0.15))
 (gr_line (start 202.438 70.866) (end 202.438 81.026) (angle 90) (layer Edge.Cuts) (width 0.15))
 (gr_line (start 199.898 68.326) (end 202.438 70.866) (angle 90) (layer Edge.Cuts) (width 0.15))
 (gr_line (start 103.378 68.326) (end 199.898 68.326) (angle 90) (layer Edge.Cuts) (width 0.15))
 (gr_line (start 103.378 121.666) (end 103.378 68.326) (angle 90) (layer Edge.Cuts) (width 0.15))
 (segment (start 143.43 118.538) (end 144.018 119.126) (width 0.25) (layer F.Cu) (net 1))
 (segment (start 143.43 102.87) (end 143.43 118.538) (width 0.25) (layer F.Cu) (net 1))
 (segment (start 142.304999 103.995001) (end 129.395001 103.995001) (width 0.25) (layer F.Cu) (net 1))
 (segment (start 143.43 102.87) (end 142.304999 103.995001) (width 0.25) (layer F.Cu) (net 1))
 (segment (start 129.395001 103.995001) (end 124.46 99.06) (width 0.25) (layer F.Cu) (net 1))
 (segment (start 124.46 99.06) (end 124.46 95.25) (width 0.25) (layer F.Cu) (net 1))
 (segment (start 124.46 95.25) (end 125.73 95.25) (width 0.25) (layer F.Cu) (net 1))
 (segment (start 125.73 95.25) (end 127 93.98) (width 0.25) (layer F.Cu) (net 1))
 (segment (start 127 93.98) (end 127 76.2) (width 0.25) (layer F.Cu) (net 1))
 (segment (start 129.794 73.406) (end 129.794 70.866) (width 0.25) (layer F.Cu) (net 1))
 (segment (start 127 76.2) (end 129.794 73.406) (width 0.25) (layer F.Cu) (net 1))
 (segment (start 166.29 105.41) (end 166.29 108.03) (width 0.25) (layer F.Cu) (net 1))
 (segment (start 166.29 108.03) (end 165.1 109.22) (width 0.25) (layer F.Cu) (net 1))
 (segment (start 165.1 109.22) (end 143.51 109.22) (width 0.25) (layer F.Cu) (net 1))
 (segment (start 145.4444 119.126) (end 144.018 119.126) (width 0.25) (layer F.Cu) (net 1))
 (segment (start 146.558 119.126) (end 145.4444 119.126) (width 0.25) (layer F.Cu) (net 1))
 (segment (start 173.99 102.87) (end 180.34 96.52) (width 0.25) (layer F.Cu) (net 1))
 (segment (start 166.29 105.41) (end 173.99 105.41) (width 0.25) (layer F.Cu) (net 1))
 (segment (start 171.45 106.68) (end 173.99 104.14) (width 0.25) (layer F.Cu) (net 1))
 (segment (start 173.99 106.68) (end 171.45 106.68) (width 0.25) (layer F.Cu) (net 1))
 (segment (start 173.99 104.14) (end 173.99 102.87) (width 0.25) (layer F.Cu) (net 1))
 (segment (start 173.99 105.41) (end 173.99 104.14) (width 0.25) (layer F.Cu) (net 1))
 (segment (start 184.07 105.41) (end 184.07 109.3) (width 0.25) (layer F.Cu) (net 1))
 (segment (start 184.07 109.3) (end 181.61 111.76) (width 0.25) (layer F.Cu) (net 1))
 (segment (start 181.61 111.76) (end 179.07 111.76) (width 0.25) (layer F.Cu) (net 1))
 (segment (start 179.07 111.76) (end 173.99 106.68) (width 0.25) (layer F.Cu) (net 1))
 (segment (start 197.358 114.046) (end 199.136 114.046) (width 0.25) (layer F.Cu) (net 1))
 (segment (start 199.136 114.046) (end 199.898 114.046) (width 0.25) (layer F.Cu) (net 1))
 (segment (start 197.358 114.046) (end 188.976 114.046) (width 0.25) (layer F.Cu) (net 1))
 (segment (start 188.976 114.046) (end 184.15 109.22) (width 0.25) (layer F.Cu) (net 1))
 (segment (start 179.07 105.41) (end 179.07 104.14) (width 0.25) (layer F.Cu) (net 88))
 (segment (start 179.07 104.14) (end 182.88 100.33) (width 0.25) (layer F.Cu) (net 88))
 (segment (start 190.5 100.33) (end 194.31 96.52) (width 0.25) (layer F.Cu) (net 88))
 (segment (start 182.88 100.33) (end 190.5 100.33) (width 0.25) (layer F.Cu) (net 88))
 (segment (start 170.18 96.52) (end 165.02 96.52) (width 0.25) (layer F.Cu) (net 2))
 (segment (start 160.02 96.52) (end 148.59 96.52) (width 0.25) (layer F.Cu) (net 89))
 (segment (start 137.16 95.25) (end 138.43 96.52) (width 0.25) (layer F.Cu) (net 90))
 (segment (start 132.08 95.25) (end 137.16 95.25) (width 0.25) (layer F.Cu) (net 90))
 (segment (start 138.43 102.87) (end 138.43 96.52) (width 0.25) (layer F.Cu) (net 90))
 (segment (start 129.54 83.82) (end 130.81 82.55) (width 0.25) (layer F.Cu) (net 91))
 (segment (start 129.54 91.44) (end 129.54 83.82) (width 0.25) (layer F.Cu) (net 91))
 (segment (start 132.08 92.71) (end 130.81 92.71) (width 0.25) (layer F.Cu) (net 91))
 (segment (start 130.81 92.71) (end 129.54 91.44) (width 0.25) (layer F.Cu) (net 91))
 (segment (start 181.61 82.55) (end 184.15 85.09) (width 0.25) (layer F.Cu) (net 91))
 (segment (start 153.59 105.41) (end 153.59 104.22) (width 0.25) (layer F.Cu) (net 91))
 (segment (start 153.59 104.22) (end 148.59 99.22) (width 0.25) (layer F.Cu) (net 91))
 (segment (start 148.59 99.22) (end 144.94 99.22) (width 0.25) (layer F.Cu) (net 91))
 (segment (start 144.94 99.22) (end 146.05 98.11) (width 0.25) (layer F.Cu) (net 91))
 (segment (start 147.790001 93.509999) (end 148.59 92.71) (width 0.25) (layer F.Cu) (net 91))
 (segment (start 146.05 95.25) (end 147.790001 93.509999) (width 0.25) (layer F.Cu) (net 91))
 (segment (start 146.05 98.11) (end 146.05 95.25) (width 0.25) (layer F.Cu) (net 91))
 (segment (start 146.05 95.25) (end 146.05 83.82) (width 0.25) (layer F.Cu) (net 91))
 (segment (start 146.05 83.82) (end 144.78 82.55) (width 0.25) (layer F.Cu) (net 91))
 (segment (start 130.81 82.55) (end 144.78 82.55) (width 0.25) (layer F.Cu) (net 91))
 (segment (start 144.78 82.55) (end 181.61 82.55) (width 0.25) (layer F.Cu) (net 91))
 (segment (start 132.08 90.17) (end 138.43 90.17) (width 0.25) (layer F.Cu) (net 92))
 (segment (start 148.59 104.16) (end 142.24 97.81) (width 0.25) (layer F.Cu) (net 92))
 (segment (start 148.59 105.41) (end 148.59 104.16) (width 0.25) (layer F.Cu) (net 92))
 (segment (start 142.24 96.52) (end 138.43 92.71) (width 0.25) (layer F.Cu) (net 92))
 (segment (start 142.24 97.81) (end 142.24 96.52) (width 0.25) (layer F.Cu) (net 92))
 (segment (start 138.43 90.17) (end 138.43 92.71) (width 0.25) (layer F.Cu) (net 92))
 (segment (start 161.29 105.41) (end 161.29 102.87) (width 0.25) (layer F.Cu) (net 93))
 (segment (start 161.29 102.87) (end 162.56 101.6) (width 0.25) (layer F.Cu) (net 93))
 (segment (start 162.56 101.6) (end 162.56 92.71) (width 0.25) (layer F.Cu) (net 93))
 (segment (start 160.02 90.17) (end 148.59 90.17) (width 0.25) (layer F.Cu) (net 93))
 (segment (start 162.56 92.71) (end 160.02 90.17) (width 0.25) (layer F.Cu) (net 93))
 (segment (start 181.61 87.63) (end 182.88 87.63) (width 0.25) (layer F.Cu) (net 94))
 (segment (start 182.88 87.63) (end 184.15 88.9) (width 0.25) (layer F.Cu) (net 94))
 (segment (start 184.15 88.9) (end 184.15 96.52) (width 0.25) (layer F.Cu) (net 94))
 (segment (start 137.16 87.63) (end 138.43 86.36) (width 0.25) (layer F.Cu) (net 95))
 (segment (start 132.08 87.63) (end 137.16 87.63) (width 0.25) (layer F.Cu) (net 95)))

